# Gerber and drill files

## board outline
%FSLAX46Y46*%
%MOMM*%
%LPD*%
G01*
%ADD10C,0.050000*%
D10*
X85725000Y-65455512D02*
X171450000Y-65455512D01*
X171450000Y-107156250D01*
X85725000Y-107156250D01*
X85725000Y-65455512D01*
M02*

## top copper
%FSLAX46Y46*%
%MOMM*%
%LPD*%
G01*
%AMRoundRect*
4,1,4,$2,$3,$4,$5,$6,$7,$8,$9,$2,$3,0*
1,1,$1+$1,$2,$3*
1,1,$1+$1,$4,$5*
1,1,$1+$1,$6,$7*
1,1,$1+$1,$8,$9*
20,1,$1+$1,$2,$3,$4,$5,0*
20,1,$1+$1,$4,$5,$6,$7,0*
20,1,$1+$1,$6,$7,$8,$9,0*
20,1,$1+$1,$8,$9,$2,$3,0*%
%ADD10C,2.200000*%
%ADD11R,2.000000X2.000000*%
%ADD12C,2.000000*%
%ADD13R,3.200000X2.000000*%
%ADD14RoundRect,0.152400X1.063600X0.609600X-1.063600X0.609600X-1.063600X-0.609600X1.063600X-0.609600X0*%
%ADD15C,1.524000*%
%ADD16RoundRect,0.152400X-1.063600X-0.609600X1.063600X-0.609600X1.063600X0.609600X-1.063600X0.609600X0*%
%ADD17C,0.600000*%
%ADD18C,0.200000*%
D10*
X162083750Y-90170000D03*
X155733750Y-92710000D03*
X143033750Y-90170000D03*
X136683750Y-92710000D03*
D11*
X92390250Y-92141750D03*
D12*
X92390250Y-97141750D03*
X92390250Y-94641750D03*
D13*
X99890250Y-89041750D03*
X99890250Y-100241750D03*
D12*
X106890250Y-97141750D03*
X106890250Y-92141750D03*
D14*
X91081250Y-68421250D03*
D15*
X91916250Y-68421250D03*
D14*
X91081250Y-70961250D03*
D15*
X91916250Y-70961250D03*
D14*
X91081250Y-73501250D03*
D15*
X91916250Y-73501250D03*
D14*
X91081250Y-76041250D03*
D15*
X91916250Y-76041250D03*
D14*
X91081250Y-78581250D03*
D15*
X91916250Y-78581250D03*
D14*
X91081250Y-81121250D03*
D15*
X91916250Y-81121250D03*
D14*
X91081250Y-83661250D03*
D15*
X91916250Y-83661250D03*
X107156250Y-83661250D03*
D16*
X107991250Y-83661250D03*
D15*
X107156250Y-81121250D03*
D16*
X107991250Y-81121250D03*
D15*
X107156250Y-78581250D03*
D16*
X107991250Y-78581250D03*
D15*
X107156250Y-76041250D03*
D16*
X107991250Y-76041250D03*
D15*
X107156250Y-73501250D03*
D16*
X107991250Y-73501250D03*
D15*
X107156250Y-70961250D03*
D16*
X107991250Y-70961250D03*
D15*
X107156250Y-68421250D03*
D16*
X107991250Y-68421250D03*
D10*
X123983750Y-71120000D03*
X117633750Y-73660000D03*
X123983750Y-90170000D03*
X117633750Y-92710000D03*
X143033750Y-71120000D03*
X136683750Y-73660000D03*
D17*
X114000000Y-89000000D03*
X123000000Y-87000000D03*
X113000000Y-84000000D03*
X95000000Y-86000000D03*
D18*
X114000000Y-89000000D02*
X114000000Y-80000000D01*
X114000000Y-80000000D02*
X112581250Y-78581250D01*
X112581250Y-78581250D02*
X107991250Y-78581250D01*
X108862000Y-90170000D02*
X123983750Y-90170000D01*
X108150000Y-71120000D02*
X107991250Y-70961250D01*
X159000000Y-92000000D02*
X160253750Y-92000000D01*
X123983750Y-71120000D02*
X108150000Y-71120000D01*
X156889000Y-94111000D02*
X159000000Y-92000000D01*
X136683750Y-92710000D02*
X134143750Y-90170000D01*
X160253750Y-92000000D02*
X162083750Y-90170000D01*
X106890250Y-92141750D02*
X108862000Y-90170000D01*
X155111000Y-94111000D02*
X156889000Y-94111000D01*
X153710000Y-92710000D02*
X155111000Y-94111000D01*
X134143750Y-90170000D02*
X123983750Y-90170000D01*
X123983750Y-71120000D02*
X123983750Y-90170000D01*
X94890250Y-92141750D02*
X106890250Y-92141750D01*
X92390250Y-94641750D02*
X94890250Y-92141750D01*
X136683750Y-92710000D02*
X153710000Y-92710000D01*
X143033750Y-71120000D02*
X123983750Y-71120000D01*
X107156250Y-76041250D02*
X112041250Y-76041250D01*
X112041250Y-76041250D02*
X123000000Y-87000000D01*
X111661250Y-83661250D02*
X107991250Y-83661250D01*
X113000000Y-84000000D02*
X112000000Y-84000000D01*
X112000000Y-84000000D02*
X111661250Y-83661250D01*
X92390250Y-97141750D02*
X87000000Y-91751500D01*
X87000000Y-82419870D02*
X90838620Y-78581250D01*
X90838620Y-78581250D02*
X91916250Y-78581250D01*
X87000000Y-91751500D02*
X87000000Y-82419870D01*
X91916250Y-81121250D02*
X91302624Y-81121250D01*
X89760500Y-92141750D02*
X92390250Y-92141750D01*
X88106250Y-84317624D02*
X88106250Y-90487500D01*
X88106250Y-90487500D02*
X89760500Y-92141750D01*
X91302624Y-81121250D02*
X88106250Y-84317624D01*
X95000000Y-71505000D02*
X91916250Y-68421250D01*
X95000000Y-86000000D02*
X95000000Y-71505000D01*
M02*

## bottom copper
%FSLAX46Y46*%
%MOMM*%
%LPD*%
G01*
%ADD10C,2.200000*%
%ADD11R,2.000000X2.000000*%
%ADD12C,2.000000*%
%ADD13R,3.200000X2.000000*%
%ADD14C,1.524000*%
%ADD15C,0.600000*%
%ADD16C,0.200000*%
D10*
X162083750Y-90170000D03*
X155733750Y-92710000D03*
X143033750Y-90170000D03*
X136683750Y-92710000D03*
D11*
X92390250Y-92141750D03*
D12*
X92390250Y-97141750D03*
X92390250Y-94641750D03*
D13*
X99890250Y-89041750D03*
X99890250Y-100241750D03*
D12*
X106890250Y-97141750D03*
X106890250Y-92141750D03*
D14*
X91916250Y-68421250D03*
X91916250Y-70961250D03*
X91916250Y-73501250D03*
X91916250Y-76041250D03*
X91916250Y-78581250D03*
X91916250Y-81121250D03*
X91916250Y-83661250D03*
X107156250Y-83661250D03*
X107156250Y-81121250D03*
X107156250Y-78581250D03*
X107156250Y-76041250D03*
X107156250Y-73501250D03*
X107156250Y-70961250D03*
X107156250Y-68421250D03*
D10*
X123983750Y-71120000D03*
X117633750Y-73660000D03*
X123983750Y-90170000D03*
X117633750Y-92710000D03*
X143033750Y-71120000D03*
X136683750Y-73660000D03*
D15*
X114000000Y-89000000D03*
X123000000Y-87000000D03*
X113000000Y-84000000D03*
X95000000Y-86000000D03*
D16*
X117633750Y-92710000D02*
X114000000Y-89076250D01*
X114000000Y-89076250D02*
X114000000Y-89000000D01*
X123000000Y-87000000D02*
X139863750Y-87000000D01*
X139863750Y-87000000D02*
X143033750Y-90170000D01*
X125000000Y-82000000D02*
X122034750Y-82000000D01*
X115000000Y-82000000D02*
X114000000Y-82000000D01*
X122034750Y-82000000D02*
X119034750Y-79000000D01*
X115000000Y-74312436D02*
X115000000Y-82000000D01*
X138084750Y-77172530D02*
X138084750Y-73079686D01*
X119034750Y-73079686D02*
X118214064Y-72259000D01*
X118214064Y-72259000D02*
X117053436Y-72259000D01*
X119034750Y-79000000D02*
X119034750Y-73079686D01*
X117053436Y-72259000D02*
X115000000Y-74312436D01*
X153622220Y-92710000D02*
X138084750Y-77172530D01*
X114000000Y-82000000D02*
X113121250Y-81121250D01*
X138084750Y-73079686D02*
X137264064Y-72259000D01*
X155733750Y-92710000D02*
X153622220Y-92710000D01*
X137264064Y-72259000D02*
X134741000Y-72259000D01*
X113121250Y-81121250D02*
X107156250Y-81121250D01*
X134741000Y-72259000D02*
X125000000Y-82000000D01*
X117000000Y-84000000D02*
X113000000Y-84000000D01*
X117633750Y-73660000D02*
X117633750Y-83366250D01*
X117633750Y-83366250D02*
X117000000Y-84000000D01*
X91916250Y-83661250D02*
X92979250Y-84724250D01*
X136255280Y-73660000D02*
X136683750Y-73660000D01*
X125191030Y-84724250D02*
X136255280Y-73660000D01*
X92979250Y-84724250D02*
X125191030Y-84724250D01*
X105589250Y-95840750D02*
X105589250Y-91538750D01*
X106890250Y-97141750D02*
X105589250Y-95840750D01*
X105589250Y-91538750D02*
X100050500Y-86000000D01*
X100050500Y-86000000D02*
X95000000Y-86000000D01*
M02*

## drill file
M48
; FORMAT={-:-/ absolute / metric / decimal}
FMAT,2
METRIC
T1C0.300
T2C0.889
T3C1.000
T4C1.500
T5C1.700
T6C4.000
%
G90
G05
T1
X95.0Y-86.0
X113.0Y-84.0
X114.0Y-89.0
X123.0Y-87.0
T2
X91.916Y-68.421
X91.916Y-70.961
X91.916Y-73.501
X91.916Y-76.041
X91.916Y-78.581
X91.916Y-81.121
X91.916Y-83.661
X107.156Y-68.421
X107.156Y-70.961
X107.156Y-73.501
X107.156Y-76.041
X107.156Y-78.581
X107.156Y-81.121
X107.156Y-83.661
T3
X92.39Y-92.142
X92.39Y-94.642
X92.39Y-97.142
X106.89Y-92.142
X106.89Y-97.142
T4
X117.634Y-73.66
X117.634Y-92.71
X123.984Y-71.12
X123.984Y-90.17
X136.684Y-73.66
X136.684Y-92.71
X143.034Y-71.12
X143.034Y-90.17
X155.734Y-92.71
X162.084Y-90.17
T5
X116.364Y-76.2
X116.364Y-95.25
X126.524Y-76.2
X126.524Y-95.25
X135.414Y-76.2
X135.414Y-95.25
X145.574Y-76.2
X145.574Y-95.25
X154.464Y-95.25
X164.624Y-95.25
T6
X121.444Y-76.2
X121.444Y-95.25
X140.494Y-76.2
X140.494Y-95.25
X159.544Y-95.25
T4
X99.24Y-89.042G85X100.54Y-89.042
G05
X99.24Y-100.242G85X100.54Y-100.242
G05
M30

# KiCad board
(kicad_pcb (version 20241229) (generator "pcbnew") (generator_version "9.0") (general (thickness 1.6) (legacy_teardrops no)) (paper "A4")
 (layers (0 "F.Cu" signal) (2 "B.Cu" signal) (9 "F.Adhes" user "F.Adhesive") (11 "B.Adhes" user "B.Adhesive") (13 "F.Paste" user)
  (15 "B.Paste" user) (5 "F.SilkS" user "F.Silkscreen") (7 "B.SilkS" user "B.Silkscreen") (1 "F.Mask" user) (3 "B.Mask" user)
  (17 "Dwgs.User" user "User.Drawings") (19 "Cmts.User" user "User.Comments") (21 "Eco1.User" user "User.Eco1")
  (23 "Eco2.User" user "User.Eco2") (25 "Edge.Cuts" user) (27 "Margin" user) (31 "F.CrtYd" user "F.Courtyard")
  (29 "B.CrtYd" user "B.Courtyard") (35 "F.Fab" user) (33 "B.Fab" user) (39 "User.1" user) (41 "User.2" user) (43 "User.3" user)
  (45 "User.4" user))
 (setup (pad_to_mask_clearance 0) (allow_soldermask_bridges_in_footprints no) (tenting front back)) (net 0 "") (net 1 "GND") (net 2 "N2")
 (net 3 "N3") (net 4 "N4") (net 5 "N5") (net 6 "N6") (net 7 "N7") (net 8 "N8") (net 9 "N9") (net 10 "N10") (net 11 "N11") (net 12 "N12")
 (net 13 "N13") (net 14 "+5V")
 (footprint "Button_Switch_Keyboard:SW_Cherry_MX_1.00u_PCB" (layer "F.Cu") (at 162.08375 90.17)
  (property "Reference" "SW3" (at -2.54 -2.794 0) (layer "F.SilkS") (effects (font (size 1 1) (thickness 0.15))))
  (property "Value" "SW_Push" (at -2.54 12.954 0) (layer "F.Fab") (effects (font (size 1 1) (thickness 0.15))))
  (pad "" np_thru_hole circle (at -7.62 5.08) (size 1.7 1.7) (drill 1.7) (layers "*.Cu" "*.Mask"))
  (pad "" np_thru_hole circle (at -2.54 5.08) (size 4 4) (drill 4) (layers "*.Cu" "*.Mask"))
  (pad "" np_thru_hole circle (at 2.54 5.08) (size 1.7 1.7) (drill 1.7) (layers "*.Cu" "*.Mask"))
  (pad "1" thru_hole circle (at 0 0) (size 2.2 2.2) (drill 1.5) (layers "*.Cu" "*.Mask") (remove_unused_layers no) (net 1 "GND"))
  (pad "2" thru_hole circle (at -6.35 2.54) (size 2.2 2.2) (drill 1.5) (layers "*.Cu" "*.Mask") (remove_unused_layers no) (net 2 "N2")))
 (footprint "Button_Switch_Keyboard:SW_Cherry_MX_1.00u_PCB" (layer "F.Cu") (at 143.03375 90.17)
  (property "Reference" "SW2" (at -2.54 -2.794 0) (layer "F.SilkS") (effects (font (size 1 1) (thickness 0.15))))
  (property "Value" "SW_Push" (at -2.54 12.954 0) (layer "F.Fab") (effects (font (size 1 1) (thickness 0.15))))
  (pad "" np_thru_hole circle (at -7.62 5.08) (size 1.7 1.7) (drill 1.7) (layers "*.Cu" "*.Mask"))
  (pad "" np_thru_hole circle (at -2.54 5.08) (size 4 4) (drill 4) (layers "*.Cu" "*.Mask"))
  (pad "" np_thru_hole circle (at 2.54 5.08) (size 1.7 1.7) (drill 1.7) (layers "*.Cu" "*.Mask"))
  (pad "1" thru_hole circle (at 0 0) (size 2.2 2.2) (drill 1.5) (layers "*.Cu" "*.Mask") (remove_unused_layers no) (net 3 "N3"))
  (pad "2" thru_hole circle (at -6.35 2.54) (size 2.2 2.2) (drill 1.5) (layers "*.Cu" "*.Mask") (remove_unused_layers no) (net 1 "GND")))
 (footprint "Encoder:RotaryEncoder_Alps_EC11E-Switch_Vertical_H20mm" (layer "F.Cu") (at 92.39025 92.14175)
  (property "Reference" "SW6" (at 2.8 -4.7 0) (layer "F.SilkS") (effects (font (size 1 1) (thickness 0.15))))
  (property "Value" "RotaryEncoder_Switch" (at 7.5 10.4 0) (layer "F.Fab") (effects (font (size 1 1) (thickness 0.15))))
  (pad "A" thru_hole rect (at 0 0) (size 2 2) (drill 1) (layers "*.Cu" "*.Mask") (remove_unused_layers no) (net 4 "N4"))
  (pad "B" thru_hole circle (at 0 5) (size 2 2) (drill 1) (layers "*.Cu" "*.Mask") (remove_unused_layers no) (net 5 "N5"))
  (pad "C" thru_hole circle (at 0 2.5) (size 2 2) (drill 1) (layers "*.Cu" "*.Mask") (remove_unused_layers no) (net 1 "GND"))
  (pad "MP" thru_hole rect (at 7.5 -3.1) (size 3.2 2) (drill oval 2.8 1.5) (layers "*.Cu" "*.Mask") (remove_unused_layers no))
  (pad "MP" thru_hole rect (at 7.5 8.1) (size 3.2 2) (drill oval 2.8 1.5) (layers "*.Cu" "*.Mask") (remove_unused_layers no))
  (pad "S1" thru_hole circle (at 14.5 5) (size 2 2) (drill 1) (layers "*.Cu" "*.Mask") (remove_unused_layers no) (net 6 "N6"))
  (pad "S2" thru_hole circle (at 14.5 0) (size 2 2) (drill 1) (layers "*.Cu" "*.Mask") (remove_unused_layers no) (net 1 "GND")))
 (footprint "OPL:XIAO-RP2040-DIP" (layer "F.Cu") (at 99.53625 76.04125)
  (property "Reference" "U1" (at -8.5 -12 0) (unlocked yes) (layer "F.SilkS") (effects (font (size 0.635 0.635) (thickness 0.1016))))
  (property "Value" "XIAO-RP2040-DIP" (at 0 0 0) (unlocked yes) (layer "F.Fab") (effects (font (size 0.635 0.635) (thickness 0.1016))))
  (pad "1" smd roundrect (at -8.455 -7.62 180) (size 2.432 1.524) (layers "F.Cu" "F.Mask") (roundrect_rratio 0.1) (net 6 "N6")
   (thermal_bridge_angle 45))
  (pad "1" thru_hole circle (at -7.62 -7.62 180) (size 1.524 1.524) (drill 0.889) (layers "*.Cu" "*.Mask") (remove_unused_layers no)
   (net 6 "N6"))
  (pad "2" smd roundrect (at -8.455 -5.08 180) (size 2.432 1.524) (layers "F.Cu" "F.Mask") (roundrect_rratio 0.1) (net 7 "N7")
   (thermal_bridge_angle 45))
  (pad "2" thru_hole circle (at -7.62 -5.08 180) (size 1.524 1.524) (drill 0.889) (layers "*.Cu" "*.Mask") (remove_unused_layers no)
   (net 7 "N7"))
  (pad "3" smd roundrect (at -8.455 -2.54 180) (size 2.432 1.524) (layers "F.Cu" "F.Mask") (roundrect_rratio 0.1) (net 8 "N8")
   (thermal_bridge_angle 45))
  (pad "3" thru_hole circle (at -7.62 -2.54 180) (size 1.524 1.524) (drill 0.889) (layers "*.Cu" "*.Mask") (remove_unused_layers no)
   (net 8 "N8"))
  (pad "4" smd roundrect (at -8.455 0 180) (size 2.432 1.524) (layers "F.Cu" "F.Mask") (roundrect_rratio 0.1) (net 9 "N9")
   (thermal_bridge_angle 45))
  (pad "4" thru_hole circle (at -7.62 0 180) (size 1.524 1.524) (drill 0.889) (layers "*.Cu" "*.Mask") (remove_unused_layers no)
   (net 9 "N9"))
  (pad "5" smd roundrect (at -8.455 2.54 180) (size 2.432 1.524) (layers "F.Cu" "F.Mask") (roundrect_rratio 0.1) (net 5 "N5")
   (thermal_bridge_angle 45))
  (pad "5" thru_hole circle (at -7.62 2.54 180) (size 1.524 1.524) (drill 0.889) (layers "*.Cu" "*.Mask") (remove_unused_layers no)
   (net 5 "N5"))
  (pad "6" smd roundrect (at -8.455 5.08 180) (size 2.432 1.524) (layers "F.Cu" "F.Mask") (roundrect_rratio 0.1) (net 4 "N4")
   (thermal_bridge_angle 45))
  (pad "6" thru_hole circle (at -7.62 5.08 180) (size 1.524 1.524) (drill 0.889) (layers "*.Cu" "*.Mask") (remove_unused_layers no)
   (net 4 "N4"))
  (pad "7" smd roundrect (at -8.455 7.62 180) (size 2.432 1.524) (layers "F.Cu" "F.Mask") (roundrect_rratio 0.1) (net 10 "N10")
   (thermal_bridge_angle 45))
  (pad "7" thru_hole circle (at -7.62 7.62 180) (size 1.524 1.524) (drill 0.889) (layers "*.Cu" "*.Mask") (remove_unused_layers no)
   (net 10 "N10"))
  (pad "8" thru_hole circle (at 7.62 7.62) (size 1.524 1.524) (drill 0.889) (layers "*.Cu" "*.Mask") (remove_unused_layers no)
   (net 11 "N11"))
  (pad "8" smd roundrect (at 8.455 7.62) (size 2.432 1.524) (layers "F.Cu" "F.Mask") (roundrect_rratio 0.1) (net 11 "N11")
   (thermal_bridge_angle 45))
  (pad "9" thru_hole circle (at 7.62 5.08) (size 1.524 1.524) (drill 0.889) (layers "*.Cu" "*.Mask") (remove_unused_layers no) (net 2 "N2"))
  (pad "9" smd roundrect (at 8.455 5.08) (size 2.432 1.524) (layers "F.Cu" "F.Mask") (roundrect_rratio 0.1) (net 2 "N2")
   (thermal_bridge_angle 45))
  (pad "10" thru_hole circle (at 7.62 2.54) (size 1.524 1.524) (drill 0.889) (layers "*.Cu" "*.Mask") (remove_unused_layers no)
   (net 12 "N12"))
  (pad "10" smd roundrect (at 8.455 2.54) (size 2.432 1.524) (layers "F.Cu" "F.Mask") (roundrect_rratio 0.1) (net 12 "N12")
   (thermal_bridge_angle 45))
  (pad "11" thru_hole circle (at 7.62 0) (size 1.524 1.524) (drill 0.889) (layers "*.Cu" "*.Mask") (remove_unused_layers no) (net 3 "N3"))
  (pad "11" smd roundrect (at 8.455 0) (size 2.432 1.524) (layers "F.Cu" "F.Mask") (roundrect_rratio 0.1) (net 3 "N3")
   (thermal_bridge_angle 45))
  (pad "12" thru_hole circle (at 7.62 -2.54) (size 1.524 1.524) (drill 0.889) (layers "*.Cu" "*.Mask") (remove_unused_layers no)
   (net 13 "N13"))
  (pad "12" smd roundrect (at 8.455 -2.54) (size 2.432 1.524) (layers "F.Cu" "F.Mask") (roundrect_rratio 0.1) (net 13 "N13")
   (thermal_bridge_angle 45))
  (pad "13" thru_hole circle (at 7.62 -5.08) (size 1.524 1.524) (drill 0.889) (layers "*.Cu" "*.Mask") (remove_unused_layers no)
   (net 1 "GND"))
  (pad "13" smd roundrect (at 8.455 -5.08) (size 2.432 1.524) (layers "F.Cu" "F.Mask") (roundrect_rratio 0.1) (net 1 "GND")
   (thermal_bridge_angle 45))
  (pad "14" thru_hole circle (at 7.62 -7.62) (size 1.524 1.524) (drill 0.889) (layers "*.Cu" "*.Mask") (remove_unused_layers no)
   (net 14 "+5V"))
  (pad "14" smd roundrect (at 8.455 -7.62) (size 2.432 1.524) (layers "F.Cu" "F.Mask") (roundrect_rratio 0.1) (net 14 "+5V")
   (thermal_bridge_angle 45)))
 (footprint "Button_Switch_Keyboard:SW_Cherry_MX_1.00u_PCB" (layer "F.Cu") (at 123.98375 71.12)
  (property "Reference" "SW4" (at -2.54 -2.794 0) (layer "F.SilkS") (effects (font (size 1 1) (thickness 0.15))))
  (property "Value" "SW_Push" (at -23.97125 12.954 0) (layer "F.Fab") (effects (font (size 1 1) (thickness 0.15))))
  (pad "" np_thru_hole circle (at -7.62 5.08) (size 1.7 1.7) (drill 1.7) (layers "*.Cu" "*.Mask"))
  (pad "" np_thru_hole circle (at -2.54 5.08) (size 4 4) (drill 4) (layers "*.Cu" "*.Mask"))
  (pad "" np_thru_hole circle (at 2.54 5.08) (size 1.7 1.7) (drill 1.7) (layers "*.Cu" "*.Mask"))
  (pad "1" thru_hole circle (at 0 0) (size 2.2 2.2) (drill 1.5) (layers "*.Cu" "*.Mask") (remove_unused_layers no) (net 1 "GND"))
  (pad "2" thru_hole circle (at -6.35 2.54) (size 2.2 2.2) (drill 1.5) (layers "*.Cu" "*.Mask") (remove_unused_layers no) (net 11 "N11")))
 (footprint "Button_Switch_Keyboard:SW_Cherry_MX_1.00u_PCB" (layer "F.Cu") (at 123.98375 90.17)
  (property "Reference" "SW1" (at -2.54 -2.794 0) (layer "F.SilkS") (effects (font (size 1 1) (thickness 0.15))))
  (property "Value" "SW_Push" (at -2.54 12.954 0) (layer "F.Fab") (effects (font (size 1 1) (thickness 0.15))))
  (pad "" np_thru_hole circle (at -7.62 5.08) (size 1.7 1.7) (drill 1.7) (layers "*.Cu" "*.Mask"))
  (pad "" np_thru_hole circle (at -2.54 5.08) (size 4 4) (drill 4) (layers "*.Cu" "*.Mask"))
  (pad "" np_thru_hole circle (at 2.54 5.08) (size 1.7 1.7) (drill 1.7) (layers "*.Cu" "*.Mask"))
  (pad "1" thru_hole circle (at 0 0) (size 2.2 2.2) (drill 1.5) (layers "*.Cu" "*.Mask") (remove_unused_layers no) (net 1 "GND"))
  (pad "2" thru_hole circle (at -6.35 2.54) (size 2.2 2.2) (drill 1.5) (layers "*.Cu" "*.Mask") (remove_unused_layers no) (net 12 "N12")))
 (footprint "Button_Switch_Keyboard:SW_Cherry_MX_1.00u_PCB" (layer "F.Cu") (at 143.03375 71.12)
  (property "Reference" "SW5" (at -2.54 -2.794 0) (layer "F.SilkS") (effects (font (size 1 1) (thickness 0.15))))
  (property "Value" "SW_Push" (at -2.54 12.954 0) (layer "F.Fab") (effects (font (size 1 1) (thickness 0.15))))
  (pad "" np_thru_hole circle (at -7.62 5.08) (size 1.7 1.7) (drill 1.7) (layers "*.Cu" "*.Mask"))
  (pad "" np_thru_hole circle (at -2.54 5.08) (size 4 4) (drill 4) (layers "*.Cu" "*.Mask"))
  (pad "" np_thru_hole circle (at 2.54 5.08) (size 1.7 1.7) (drill 1.7) (layers "*.Cu" "*.Mask"))
  (pad "1" thru_hole circle (at 0 0) (size 2.2 2.2) (drill 1.5) (layers "*.Cu" "*.Mask") (remove_unused_layers no) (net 1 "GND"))
  (pad "2" thru_hole circle (at -6.35 2.54) (size 2.2 2.2) (drill 1.5) (layers "*.Cu" "*.Mask") (remove_unused_layers no) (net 10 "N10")))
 (gr_rect (start 85.725 65.455512) (end 171.45 107.15625) (stroke (width 0.05) (type default)) (fill no) (layer "Edge.Cuts"))
 (segment (start 114 89) (end 114 80) (width 0.2) (layer "F.Cu") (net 12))
 (segment (start 114 80) (end 112.58125 78.58125) (width 0.2) (layer "F.Cu") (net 12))
 (segment (start 112.58125 78.58125) (end 107.99125 78.58125) (width 0.2) (layer "F.Cu") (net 12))
 (via (at 114 89) (size 0.6) (drill 0.3) (layers "F.Cu" "B.Cu") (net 12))
 (segment (start 117.63375 92.71) (end 114 89.07625) (width 0.2) (layer "B.Cu") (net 12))
 (segment (start 114 89.07625) (end 114 89) (width 0.2) (layer "B.Cu") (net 12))
 (segment (start 108.862 90.17) (end 123.98375 90.17) (width 0.2) (layer "F.Cu") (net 1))
 (segment (start 108.15 71.12) (end 107.99125 70.96125) (width 0.2) (layer "F.Cu") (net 1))
 (segment (start 159 92) (end 160.25375 92) (width 0.2) (layer "F.Cu") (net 1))
 (segment (start 123.98375 71.12) (end 108.15 71.12) (width 0.2) (layer "F.Cu") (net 1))
 (segment (start 156.889 94.111) (end 159 92) (width 0.2) (layer "F.Cu") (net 1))
 (segment (start 136.68375 92.71) (end 134.14375 90.17) (width 0.2) (layer "F.Cu") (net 1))
 (segment (start 160.25375 92) (end 162.08375 90.17) (width 0.2) (layer "F.Cu") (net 1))
 (segment (start 106.89025 92.14175) (end 108.862 90.17) (width 0.2) (layer "F.Cu") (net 1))
 (segment (start 155.111 94.111) (end 156.889 94.111) (width 0.2) (layer "F.Cu") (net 1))
 (segment (start 153.71 92.71) (end 155.111 94.111) (width 0.2) (layer "F.Cu") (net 1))
 (segment (start 134.14375 90.17) (end 123.98375 90.17) (width 0.2) (layer "F.Cu") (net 1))
 (segment (start 123.98375 71.12) (end 123.98375 90.17) (width 0.2) (layer "F.Cu") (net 1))
 (segment (start 94.89025 92.14175) (end 106.89025 92.14175) (width 0.2) (layer "F.Cu") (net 1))
 (segment (start 92.39025 94.64175) (end 94.89025 92.14175) (width 0.2) (layer "F.Cu") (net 1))
 (segment (start 136.68375 92.71) (end 153.71 92.71) (width 0.2) (layer "F.Cu") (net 1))
 (segment (start 143.03375 71.12) (end 123.98375 71.12) (width 0.2) (layer "F.Cu") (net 1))
 (segment (start 107.15625 76.04125) (end 112.04125 76.04125) (width 0.2) (layer "F.Cu") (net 3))
 (segment (start 112.04125 76.04125) (end 123 87) (width 0.2) (layer "F.Cu") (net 3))
 (via (at 123 87) (size 0.6) (drill 0.3) (layers "F.Cu" "B.Cu") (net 3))
 (segment (start 123 87) (end 139.86375 87) (width 0.2) (layer "B.Cu") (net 3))
 (segment (start 139.86375 87) (end 143.03375 90.17) (width 0.2) (layer "B.Cu") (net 3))
 (segment (start 125 82) (end 122.03475 82) (width 0.2) (layer "B.Cu") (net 2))
 (segment (start 115 82) (end 114 82) (width 0.2) (layer "B.Cu") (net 2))
 (segment (start 122.03475 82) (end 119.03475 79) (width 0.2) (layer "B.Cu") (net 2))
 (segment (start 115 74.312436) (end 115 82) (width 0.2) (layer "B.Cu") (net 2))
 (segment (start 138.08475 77.17253) (end 138.08475 73.079686) (width 0.2) (layer "B.Cu") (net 2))
 (segment (start 119.03475 73.079686) (end 118.214064 72.259) (width 0.2) (layer "B.Cu") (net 2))
 (segment (start 118.214064 72.259) (end 117.053436 72.259) (width 0.2) (layer "B.Cu") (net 2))
 (segment (start 119.03475 79) (end 119.03475 73.079686) (width 0.2) (layer "B.Cu") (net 2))
 (segment (start 117.053436 72.259) (end 115 74.312436) (width 0.2) (layer "B.Cu") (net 2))
 (segment (start 153.62222 92.71) (end 138.08475 77.17253) (width 0.2) (layer "B.Cu") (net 2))
 (segment (start 114 82) (end 113.12125 81.12125) (width 0.2) (layer "B.Cu") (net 2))
 (segment (start 138.08475 73.079686) (end 137.264064 72.259) (width 0.2) (layer "B.Cu") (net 2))
 (segment (start 155.73375 92.71) (end 153.62222 92.71) (width 0.2) (layer "B.Cu") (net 2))
 (segment (start 137.264064 72.259) (end 134.741 72.259) (width 0.2) (layer "B.Cu") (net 2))
 (segment (start 113.12125 81.12125) (end 107.15625 81.12125) (width 0.2) (layer "B.Cu") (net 2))
 (segment (start 134.741 72.259) (end 125 82) (width 0.2) (layer "B.Cu") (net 2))
 (segment (start 111.66125 83.66125) (end 107.99125 83.66125) (width 0.2) (layer "F.Cu") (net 11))
 (segment (start 113 84) (end 112 84) (width 0.2) (layer "F.Cu") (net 11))
 (segment (start 112 84) (end 111.66125 83.66125) (width 0.2) (layer "F.Cu") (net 11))
 (via (at 113 84) (size 0.6) (drill 0.3) (layers "F.Cu" "B.Cu") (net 11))
 (segment (start 117 84) (end 113 84) (width 0.2) (layer "B.Cu") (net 11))
 (segment (start 117.63375 73.66) (end 117.63375 83.36625) (width 0.2) (layer "B.Cu") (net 11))
 (segment (start 117.63375 83.36625) (end 117 84) (width 0.2) (layer "B.Cu") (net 11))
 (segment (start 91.91625 83.66125) (end 92.97925 84.72425) (width 0.2) (layer "B.Cu") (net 10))
 (segment (start 136.25528 73.66) (end 136.68375 73.66) (width 0.2) (layer "B.Cu") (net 10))
 (segment (start 125.19103 84.72425) (end 136.25528 73.66) (width 0.2) (layer "B.Cu") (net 10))
 (segment (start 92.97925 84.72425) (end 125.19103 84.72425) (width 0.2) (layer "B.Cu") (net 10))
 (segment (start 92.39025 97.14175) (end 87 91.7515) (width 0.2) (layer "F.Cu") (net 5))
 (segment (start 87 82.41987) (end 90.83862 78.58125) (width 0.2) (layer "F.Cu") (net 5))
 (segment (start 90.83862 78.58125) (end 91.91625 78.58125) (width 0.2) (layer "F.Cu") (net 5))
 (segment (start 87 91.7515) (end 87 82.41987) (width 0.2) (layer "F.Cu") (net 5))
 (segment (start 91.91625 81.12125) (end 91.302624 81.12125) (width 0.2) (layer "F.Cu") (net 4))
 (segment (start 89.7605 92.14175) (end 92.39025 92.14175) (width 0.2) (layer "F.Cu") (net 4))
 (segment (start 88.10625 84.317624) (end 88.10625 90.4875) (width 0.2) (layer "F.Cu") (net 4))
 (segment (start 88.10625 90.4875) (end 89.7605 92.14175) (width 0.2) (layer "F.Cu") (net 4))
 (segment (start 91.302624 81.12125) (end 88.10625 84.317624) (width 0.2) (layer "F.Cu") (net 4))
 (segment (start 95 71.505) (end 91.91625 68.42125) (width 0.2) (layer "F.Cu") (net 6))
 (segment (start 95 86) (end 95 71.505) (width 0.2) (layer "F.Cu") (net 6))
 (via (at 95 86) (size 0.6) (drill 0.3) (layers "F.Cu" "B.Cu") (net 6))
 (segment (start 105.58925 95.84075) (end 105.58925 91.53875) (width 0.2) (layer "B.Cu") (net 6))
 (segment (start 106.89025 97.14175) (end 105.58925 95.84075) (width 0.2) (layer "B.Cu") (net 6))
 (segment (start 105.58925 91.53875) (end 100.0505 86) (width 0.2) (layer "B.Cu") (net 6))
 (segment (start 100.0505 86) (end 95 86) (width 0.2) (layer "B.Cu") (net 6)))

